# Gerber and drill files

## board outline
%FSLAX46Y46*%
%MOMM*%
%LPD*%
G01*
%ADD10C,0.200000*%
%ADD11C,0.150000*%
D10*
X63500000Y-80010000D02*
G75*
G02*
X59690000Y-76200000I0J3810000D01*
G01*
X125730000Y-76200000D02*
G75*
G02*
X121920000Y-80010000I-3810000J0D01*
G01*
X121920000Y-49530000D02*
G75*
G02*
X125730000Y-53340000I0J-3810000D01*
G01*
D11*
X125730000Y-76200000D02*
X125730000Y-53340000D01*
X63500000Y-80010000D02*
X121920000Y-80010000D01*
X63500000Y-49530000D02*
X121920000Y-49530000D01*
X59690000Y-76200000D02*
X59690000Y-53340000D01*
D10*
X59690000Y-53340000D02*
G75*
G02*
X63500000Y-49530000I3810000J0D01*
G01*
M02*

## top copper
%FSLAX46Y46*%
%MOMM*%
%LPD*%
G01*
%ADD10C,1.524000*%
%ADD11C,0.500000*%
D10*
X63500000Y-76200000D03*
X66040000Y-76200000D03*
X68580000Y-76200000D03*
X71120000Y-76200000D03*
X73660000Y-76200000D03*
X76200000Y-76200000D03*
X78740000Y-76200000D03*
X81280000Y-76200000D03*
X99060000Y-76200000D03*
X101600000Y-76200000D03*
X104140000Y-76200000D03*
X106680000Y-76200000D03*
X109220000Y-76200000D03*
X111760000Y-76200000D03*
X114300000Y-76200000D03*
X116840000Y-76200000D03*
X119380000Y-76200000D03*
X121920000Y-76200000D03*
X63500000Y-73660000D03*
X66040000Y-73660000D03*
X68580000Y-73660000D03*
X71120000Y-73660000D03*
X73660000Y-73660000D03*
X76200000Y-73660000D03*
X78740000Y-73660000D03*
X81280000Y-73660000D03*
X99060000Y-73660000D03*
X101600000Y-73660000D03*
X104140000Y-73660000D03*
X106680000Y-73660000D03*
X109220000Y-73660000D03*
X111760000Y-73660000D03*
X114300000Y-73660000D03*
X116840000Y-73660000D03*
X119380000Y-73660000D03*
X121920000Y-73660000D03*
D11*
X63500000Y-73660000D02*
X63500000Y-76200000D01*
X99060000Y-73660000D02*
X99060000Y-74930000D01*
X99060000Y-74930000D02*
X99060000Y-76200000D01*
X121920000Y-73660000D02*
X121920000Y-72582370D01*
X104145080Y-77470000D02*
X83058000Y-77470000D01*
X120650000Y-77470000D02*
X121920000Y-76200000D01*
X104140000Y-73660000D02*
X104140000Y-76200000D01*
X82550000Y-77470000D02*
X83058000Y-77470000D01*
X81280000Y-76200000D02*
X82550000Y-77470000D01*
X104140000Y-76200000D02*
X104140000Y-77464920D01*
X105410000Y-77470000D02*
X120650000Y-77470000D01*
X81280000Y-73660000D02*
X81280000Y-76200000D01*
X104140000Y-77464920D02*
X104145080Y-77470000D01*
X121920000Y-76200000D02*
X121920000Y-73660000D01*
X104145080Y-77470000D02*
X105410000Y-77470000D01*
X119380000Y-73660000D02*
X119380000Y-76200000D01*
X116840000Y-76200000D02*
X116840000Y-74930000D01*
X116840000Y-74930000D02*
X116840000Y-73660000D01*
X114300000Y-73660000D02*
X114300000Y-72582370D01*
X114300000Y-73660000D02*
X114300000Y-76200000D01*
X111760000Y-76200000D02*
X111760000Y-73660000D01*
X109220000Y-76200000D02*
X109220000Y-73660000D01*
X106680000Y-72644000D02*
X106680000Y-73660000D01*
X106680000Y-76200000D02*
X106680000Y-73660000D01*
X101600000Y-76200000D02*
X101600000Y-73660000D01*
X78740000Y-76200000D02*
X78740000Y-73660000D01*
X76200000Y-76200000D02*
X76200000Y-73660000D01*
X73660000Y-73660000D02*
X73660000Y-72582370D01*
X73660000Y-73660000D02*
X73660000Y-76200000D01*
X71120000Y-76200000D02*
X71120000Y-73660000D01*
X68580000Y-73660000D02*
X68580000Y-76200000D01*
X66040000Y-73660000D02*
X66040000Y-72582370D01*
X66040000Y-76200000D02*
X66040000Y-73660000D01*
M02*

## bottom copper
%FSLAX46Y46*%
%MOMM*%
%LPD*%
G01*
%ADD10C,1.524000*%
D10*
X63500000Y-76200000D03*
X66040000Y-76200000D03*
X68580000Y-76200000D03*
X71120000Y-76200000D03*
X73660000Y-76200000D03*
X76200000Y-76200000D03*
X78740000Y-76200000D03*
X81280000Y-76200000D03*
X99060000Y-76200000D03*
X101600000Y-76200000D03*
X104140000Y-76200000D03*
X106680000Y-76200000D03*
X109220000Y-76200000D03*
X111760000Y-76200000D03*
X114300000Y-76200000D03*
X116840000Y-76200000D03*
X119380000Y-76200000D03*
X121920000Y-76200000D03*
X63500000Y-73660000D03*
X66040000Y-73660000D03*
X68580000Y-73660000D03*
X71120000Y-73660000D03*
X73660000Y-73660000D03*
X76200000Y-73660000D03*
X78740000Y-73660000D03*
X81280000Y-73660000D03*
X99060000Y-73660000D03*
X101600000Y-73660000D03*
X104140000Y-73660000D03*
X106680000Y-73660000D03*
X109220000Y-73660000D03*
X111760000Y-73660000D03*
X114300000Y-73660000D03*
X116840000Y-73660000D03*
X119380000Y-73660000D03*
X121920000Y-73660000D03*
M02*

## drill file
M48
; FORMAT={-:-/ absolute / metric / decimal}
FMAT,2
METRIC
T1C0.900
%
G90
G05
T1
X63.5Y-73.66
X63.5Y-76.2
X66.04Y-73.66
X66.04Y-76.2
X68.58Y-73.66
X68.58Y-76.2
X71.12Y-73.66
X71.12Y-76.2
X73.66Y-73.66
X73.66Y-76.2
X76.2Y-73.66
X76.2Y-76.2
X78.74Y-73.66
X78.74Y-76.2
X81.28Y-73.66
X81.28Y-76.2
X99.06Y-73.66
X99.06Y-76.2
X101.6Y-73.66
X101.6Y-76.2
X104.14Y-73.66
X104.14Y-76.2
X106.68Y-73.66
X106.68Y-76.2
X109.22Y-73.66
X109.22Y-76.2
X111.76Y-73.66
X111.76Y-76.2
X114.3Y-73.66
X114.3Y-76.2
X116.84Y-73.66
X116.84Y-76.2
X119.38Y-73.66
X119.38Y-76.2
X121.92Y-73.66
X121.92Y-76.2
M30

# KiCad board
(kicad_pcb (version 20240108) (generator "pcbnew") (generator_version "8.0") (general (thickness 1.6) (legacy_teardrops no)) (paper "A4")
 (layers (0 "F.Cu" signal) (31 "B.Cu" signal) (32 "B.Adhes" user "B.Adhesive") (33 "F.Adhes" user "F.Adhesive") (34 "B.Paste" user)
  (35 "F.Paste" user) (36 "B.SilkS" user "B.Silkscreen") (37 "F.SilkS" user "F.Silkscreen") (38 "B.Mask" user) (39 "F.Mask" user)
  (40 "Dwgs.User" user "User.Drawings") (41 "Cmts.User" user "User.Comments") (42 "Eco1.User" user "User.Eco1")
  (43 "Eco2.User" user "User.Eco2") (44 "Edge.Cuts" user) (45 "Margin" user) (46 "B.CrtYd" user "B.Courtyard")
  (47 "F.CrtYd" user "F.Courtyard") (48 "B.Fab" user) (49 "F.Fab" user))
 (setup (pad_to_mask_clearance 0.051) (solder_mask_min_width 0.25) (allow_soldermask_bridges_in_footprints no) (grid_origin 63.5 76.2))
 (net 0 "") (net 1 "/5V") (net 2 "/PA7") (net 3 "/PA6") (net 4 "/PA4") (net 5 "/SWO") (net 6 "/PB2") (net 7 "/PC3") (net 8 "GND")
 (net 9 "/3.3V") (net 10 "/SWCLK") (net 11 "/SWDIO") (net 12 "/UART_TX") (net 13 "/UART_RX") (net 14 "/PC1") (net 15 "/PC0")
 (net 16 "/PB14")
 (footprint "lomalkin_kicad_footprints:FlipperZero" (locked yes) (layer "F.Cu") (at 90.17 76.2)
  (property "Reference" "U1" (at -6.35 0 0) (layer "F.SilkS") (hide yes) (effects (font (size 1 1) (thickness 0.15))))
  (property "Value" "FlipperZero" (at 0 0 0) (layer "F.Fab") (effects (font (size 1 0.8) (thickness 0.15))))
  (pad "1" thru_hole circle (at -26.67 0 270) (size 1.524 1.524) (drill 0.9) (layers "*.Cu" "*.Mask") (remove_unused_layers no)
   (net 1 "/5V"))
  (pad "2" thru_hole circle (at -24.13 0 270) (size 1.524 1.524) (drill 0.9) (layers "*.Cu" "*.Mask") (remove_unused_layers no)
   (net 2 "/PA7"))
  (pad "3" thru_hole circle (at -21.59 0 270) (size 1.524 1.524) (drill 0.9) (layers "*.Cu" "*.Mask") (remove_unused_layers no)
   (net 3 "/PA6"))
  (pad "4" thru_hole circle (at -19.05 0 270) (size 1.524 1.524) (drill 0.9) (layers "*.Cu" "*.Mask") (remove_unused_layers no)
   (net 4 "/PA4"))
  (pad "5" thru_hole circle (at -16.51 0 270) (size 1.524 1.524) (drill 0.9) (layers "*.Cu" "*.Mask") (remove_unused_layers no)
   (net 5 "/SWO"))
  (pad "6" thru_hole circle (at -13.97 0 270) (size 1.524 1.524) (drill 0.9) (layers "*.Cu" "*.Mask") (remove_unused_layers no)
   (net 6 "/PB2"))
  (pad "7" thru_hole circle (at -11.43 0 270) (size 1.524 1.524) (drill 0.9) (layers "*.Cu" "*.Mask") (remove_unused_layers no)
   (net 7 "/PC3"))
  (pad "8" thru_hole circle (at -8.89 0 270) (size 1.524 1.524) (drill 0.9) (layers "*.Cu" "*.Mask") (remove_unused_layers no) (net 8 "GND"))
  (pad "9" thru_hole circle (at 8.89 0 270) (size 1.524 1.524) (drill 0.9) (layers "*.Cu" "*.Mask") (remove_unused_layers no)
   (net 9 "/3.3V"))
  (pad "10" thru_hole circle (at 11.43 0 270) (size 1.524 1.524) (drill 0.9) (layers "*.Cu" "*.Mask") (remove_unused_layers no)
   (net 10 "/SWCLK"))
  (pad "11" thru_hole circle (at 13.97 0 270) (size 1.524 1.524) (drill 0.9) (layers "*.Cu" "*.Mask") (remove_unused_layers no)
   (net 8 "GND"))
  (pad "12" thru_hole circle (at 16.51 0 270) (size 1.524 1.524) (drill 0.9) (layers "*.Cu" "*.Mask") (remove_unused_layers no)
   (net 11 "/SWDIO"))
  (pad "13" thru_hole circle (at 19.05 0 270) (size 1.524 1.524) (drill 0.9) (layers "*.Cu" "*.Mask") (remove_unused_layers no)
   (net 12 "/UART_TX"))
  (pad "14" thru_hole circle (at 21.59 0 270) (size 1.524 1.524) (drill 0.9) (layers "*.Cu" "*.Mask") (remove_unused_layers no)
   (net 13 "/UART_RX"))
  (pad "15" thru_hole circle (at 24.13 0 270) (size 1.524 1.524) (drill 0.9) (layers "*.Cu" "*.Mask") (remove_unused_layers no)
   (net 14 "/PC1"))
  (pad "16" thru_hole circle (at 26.67 0 270) (size 1.524 1.524) (drill 0.9) (layers "*.Cu" "*.Mask") (remove_unused_layers no)
   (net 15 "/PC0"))
  (pad "17" thru_hole circle (at 29.21 0 270) (size 1.524 1.524) (drill 0.9) (layers "*.Cu" "*.Mask") (remove_unused_layers no)
   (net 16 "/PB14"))
  (pad "18" thru_hole circle (at 31.75 0 270) (size 1.524 1.524) (drill 0.9) (layers "*.Cu" "*.Mask") (remove_unused_layers no)
   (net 8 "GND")))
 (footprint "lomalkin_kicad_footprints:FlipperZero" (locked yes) (layer "F.Cu") (at 90.17 73.66)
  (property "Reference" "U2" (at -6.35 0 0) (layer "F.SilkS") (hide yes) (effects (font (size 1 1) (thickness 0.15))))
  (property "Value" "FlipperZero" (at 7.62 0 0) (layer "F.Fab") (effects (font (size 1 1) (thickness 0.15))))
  (pad "1" thru_hole circle (at -26.67 0 270) (size 1.524 1.524) (drill 0.9) (layers "*.Cu" "*.Mask") (remove_unused_layers no)
   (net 1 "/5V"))
  (pad "2" thru_hole circle (at -24.13 0 270) (size 1.524 1.524) (drill 0.9) (layers "*.Cu" "*.Mask") (remove_unused_layers no)
   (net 2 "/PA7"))
  (pad "3" thru_hole circle (at -21.59 0 270) (size 1.524 1.524) (drill 0.9) (layers "*.Cu" "*.Mask") (remove_unused_layers no)
   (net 3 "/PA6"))
  (pad "4" thru_hole circle (at -19.05 0 270) (size 1.524 1.524) (drill 0.9) (layers "*.Cu" "*.Mask") (remove_unused_layers no)
   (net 4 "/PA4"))
  (pad "5" thru_hole circle (at -16.51 0 270) (size 1.524 1.524) (drill 0.9) (layers "*.Cu" "*.Mask") (remove_unused_layers no)
   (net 5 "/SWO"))
  (pad "6" thru_hole circle (at -13.97 0 270) (size 1.524 1.524) (drill 0.9) (layers "*.Cu" "*.Mask") (remove_unused_layers no)
   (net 6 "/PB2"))
  (pad "7" thru_hole circle (at -11.43 0 270) (size 1.524 1.524) (drill 0.9) (layers "*.Cu" "*.Mask") (remove_unused_layers no)
   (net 7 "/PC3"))
  (pad "8" thru_hole circle (at -8.89 0 270) (size 1.524 1.524) (drill 0.9) (layers "*.Cu" "*.Mask") (remove_unused_layers no) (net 8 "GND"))
  (pad "9" thru_hole circle (at 8.89 0 270) (size 1.524 1.524) (drill 0.9) (layers "*.Cu" "*.Mask") (remove_unused_layers no)
   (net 9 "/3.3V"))
  (pad "10" thru_hole circle (at 11.43 0 270) (size 1.524 1.524) (drill 0.9) (layers "*.Cu" "*.Mask") (remove_unused_layers no)
   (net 10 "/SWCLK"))
  (pad "11" thru_hole circle (at 13.97 0 270) (size 1.524 1.524) (drill 0.9) (layers "*.Cu" "*.Mask") (remove_unused_layers no)
   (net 8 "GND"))
  (pad "12" thru_hole circle (at 16.51 0 270) (size 1.524 1.524) (drill 0.9) (layers "*.Cu" "*.Mask") (remove_unused_layers no)
   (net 11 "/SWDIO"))
  (pad "13" thru_hole circle (at 19.05 0 270) (size 1.524 1.524) (drill 0.9) (layers "*.Cu" "*.Mask") (remove_unused_layers no)
   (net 12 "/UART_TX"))
  (pad "14" thru_hole circle (at 21.59 0 270) (size 1.524 1.524) (drill 0.9) (layers "*.Cu" "*.Mask") (remove_unused_layers no)
   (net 13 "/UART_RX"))
  (pad "15" thru_hole circle (at 24.13 0 270) (size 1.524 1.524) (drill 0.9) (layers "*.Cu" "*.Mask") (remove_unused_layers no)
   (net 14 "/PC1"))
  (pad "16" thru_hole circle (at 26.67 0 270) (size 1.524 1.524) (drill 0.9) (layers "*.Cu" "*.Mask") (remove_unused_layers no)
   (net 15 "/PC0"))
  (pad "17" thru_hole circle (at 29.21 0 270) (size 1.524 1.524) (drill 0.9) (layers "*.Cu" "*.Mask") (remove_unused_layers no)
   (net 16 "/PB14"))
  (pad "18" thru_hole circle (at 31.75 0 270) (size 1.524 1.524) (drill 0.9) (layers "*.Cu" "*.Mask") (remove_unused_layers no)
   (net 8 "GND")))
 (gr_arc (start 63.5 80.01) (mid 60.805923 78.894077) (end 59.69 76.2) (stroke (width 0.2) (type solid)) (layer "Edge.Cuts"))
 (gr_arc (start 125.73 76.2) (mid 124.614077 78.894077) (end 121.92 80.01) (stroke (width 0.2) (type solid)) (layer "Edge.Cuts"))
 (gr_arc (start 121.92 49.53) (mid 124.614077 50.645923) (end 125.73 53.34) (stroke (width 0.2) (type solid)) (layer "Edge.Cuts"))
 (gr_line (start 125.73 76.2) (end 125.73 53.34) (stroke (width 0.15) (type solid)) (layer "Edge.Cuts"))
 (gr_line (start 63.5 80.01) (end 121.92 80.01) (stroke (width 0.15) (type solid)) (layer "Edge.Cuts"))
 (gr_line (start 63.5 49.53) (end 121.92 49.53) (stroke (width 0.15) (type solid)) (layer "Edge.Cuts"))
 (gr_line (start 59.69 76.2) (end 59.69 53.34) (stroke (width 0.15) (type solid)) (layer "Edge.Cuts"))
 (gr_arc (start 59.69 53.34) (mid 60.805923 50.645923) (end 63.5 49.53) (stroke (width 0.2) (type solid)) (layer "Edge.Cuts"))
 (segment (start 63.5 73.66) (end 63.5 76.2) (width 0.5) (layer "F.Cu") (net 1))
 (segment (start 99.06 73.66) (end 99.06 74.93) (width 0.5) (layer "F.Cu") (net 9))
 (segment (start 99.06 74.93) (end 99.06 76.2) (width 0.5) (layer "F.Cu") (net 9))
 (segment (start 121.92 73.66) (end 121.92 72.58237) (width 0.5) (layer "F.Cu") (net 8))
 (segment (start 104.14508 77.47) (end 83.058 77.47) (width 0.5) (layer "F.Cu") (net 8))
 (segment (start 120.65 77.47) (end 121.92 76.2) (width 0.5) (layer "F.Cu") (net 8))
 (segment (start 104.14 73.66) (end 104.14 76.2) (width 0.5) (layer "F.Cu") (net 8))
 (segment (start 82.55 77.47) (end 83.058 77.47) (width 0.5) (layer "F.Cu") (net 8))
 (segment (start 81.28 76.2) (end 82.55 77.47) (width 0.5) (layer "F.Cu") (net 8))
 (segment (start 104.14 76.2) (end 104.14 77.46492) (width 0.5) (layer "F.Cu") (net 8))
 (segment (start 105.41 77.47) (end 120.65 77.47) (width 0.5) (layer "F.Cu") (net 8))
 (segment (start 81.28 73.66) (end 81.28 76.2) (width 0.5) (layer "F.Cu") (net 8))
 (segment (start 104.14 77.46492) (end 104.14508 77.47) (width 0.5) (layer "F.Cu") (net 8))
 (segment (start 121.92 76.2) (end 121.92 73.66) (width 0.5) (layer "F.Cu") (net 8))
 (segment (start 104.14508 77.47) (end 105.41 77.47) (width 0.5) (layer "F.Cu") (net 8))
 (segment (start 119.38 73.66) (end 119.38 76.2) (width 0.5) (layer "F.Cu") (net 16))
 (segment (start 116.84 76.2) (end 116.84 74.93) (width 0.5) (layer "F.Cu") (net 15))
 (segment (start 116.84 74.93) (end 116.84 73.66) (width 0.5) (layer "F.Cu") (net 15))
 (segment (start 114.3 73.66) (end 114.3 72.58237) (width 0.5) (layer "F.Cu") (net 14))
 (segment (start 114.3 73.66) (end 114.3 76.2) (width 0.5) (layer "F.Cu") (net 14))
 (segment (start 111.76 76.2) (end 111.76 73.66) (width 0.5) (layer "F.Cu") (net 13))
 (segment (start 109.22 76.2) (end 109.22 73.66) (width 0.5) (layer "F.Cu") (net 12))
 (segment (start 106.68 72.644) (end 106.68 73.66) (width 0.5) (layer "F.Cu") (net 11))
 (segment (start 106.68 76.2) (end 106.68 73.66) (width 0.5) (layer "F.Cu") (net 11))
 (segment (start 101.6 76.2) (end 101.6 73.66) (width 0.5) (layer "F.Cu") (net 10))
 (segment (start 78.74 76.2) (end 78.74 73.66) (width 0.5) (layer "F.Cu") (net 7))
 (segment (start 76.2 76.2) (end 76.2 73.66) (width 0.5) (layer "F.Cu") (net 6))
 (segment (start 73.66 73.66) (end 73.66 72.58237) (width 0.5) (layer "F.Cu") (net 5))
 (segment (start 73.66 73.66) (end 73.66 76.2) (width 0.5) (layer "F.Cu") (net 5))
 (segment (start 71.12 76.2) (end 71.12 73.66) (width 0.5) (layer "F.Cu") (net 4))
 (segment (start 68.58 73.66) (end 68.58 76.2) (width 0.5) (layer "F.Cu") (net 3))
 (segment (start 66.04 73.66) (end 66.04 72.58237) (width 0.5) (layer "F.Cu") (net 2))
 (segment (start 66.04 76.2) (end 66.04 73.66) (width 0.5) (layer "F.Cu") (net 2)))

